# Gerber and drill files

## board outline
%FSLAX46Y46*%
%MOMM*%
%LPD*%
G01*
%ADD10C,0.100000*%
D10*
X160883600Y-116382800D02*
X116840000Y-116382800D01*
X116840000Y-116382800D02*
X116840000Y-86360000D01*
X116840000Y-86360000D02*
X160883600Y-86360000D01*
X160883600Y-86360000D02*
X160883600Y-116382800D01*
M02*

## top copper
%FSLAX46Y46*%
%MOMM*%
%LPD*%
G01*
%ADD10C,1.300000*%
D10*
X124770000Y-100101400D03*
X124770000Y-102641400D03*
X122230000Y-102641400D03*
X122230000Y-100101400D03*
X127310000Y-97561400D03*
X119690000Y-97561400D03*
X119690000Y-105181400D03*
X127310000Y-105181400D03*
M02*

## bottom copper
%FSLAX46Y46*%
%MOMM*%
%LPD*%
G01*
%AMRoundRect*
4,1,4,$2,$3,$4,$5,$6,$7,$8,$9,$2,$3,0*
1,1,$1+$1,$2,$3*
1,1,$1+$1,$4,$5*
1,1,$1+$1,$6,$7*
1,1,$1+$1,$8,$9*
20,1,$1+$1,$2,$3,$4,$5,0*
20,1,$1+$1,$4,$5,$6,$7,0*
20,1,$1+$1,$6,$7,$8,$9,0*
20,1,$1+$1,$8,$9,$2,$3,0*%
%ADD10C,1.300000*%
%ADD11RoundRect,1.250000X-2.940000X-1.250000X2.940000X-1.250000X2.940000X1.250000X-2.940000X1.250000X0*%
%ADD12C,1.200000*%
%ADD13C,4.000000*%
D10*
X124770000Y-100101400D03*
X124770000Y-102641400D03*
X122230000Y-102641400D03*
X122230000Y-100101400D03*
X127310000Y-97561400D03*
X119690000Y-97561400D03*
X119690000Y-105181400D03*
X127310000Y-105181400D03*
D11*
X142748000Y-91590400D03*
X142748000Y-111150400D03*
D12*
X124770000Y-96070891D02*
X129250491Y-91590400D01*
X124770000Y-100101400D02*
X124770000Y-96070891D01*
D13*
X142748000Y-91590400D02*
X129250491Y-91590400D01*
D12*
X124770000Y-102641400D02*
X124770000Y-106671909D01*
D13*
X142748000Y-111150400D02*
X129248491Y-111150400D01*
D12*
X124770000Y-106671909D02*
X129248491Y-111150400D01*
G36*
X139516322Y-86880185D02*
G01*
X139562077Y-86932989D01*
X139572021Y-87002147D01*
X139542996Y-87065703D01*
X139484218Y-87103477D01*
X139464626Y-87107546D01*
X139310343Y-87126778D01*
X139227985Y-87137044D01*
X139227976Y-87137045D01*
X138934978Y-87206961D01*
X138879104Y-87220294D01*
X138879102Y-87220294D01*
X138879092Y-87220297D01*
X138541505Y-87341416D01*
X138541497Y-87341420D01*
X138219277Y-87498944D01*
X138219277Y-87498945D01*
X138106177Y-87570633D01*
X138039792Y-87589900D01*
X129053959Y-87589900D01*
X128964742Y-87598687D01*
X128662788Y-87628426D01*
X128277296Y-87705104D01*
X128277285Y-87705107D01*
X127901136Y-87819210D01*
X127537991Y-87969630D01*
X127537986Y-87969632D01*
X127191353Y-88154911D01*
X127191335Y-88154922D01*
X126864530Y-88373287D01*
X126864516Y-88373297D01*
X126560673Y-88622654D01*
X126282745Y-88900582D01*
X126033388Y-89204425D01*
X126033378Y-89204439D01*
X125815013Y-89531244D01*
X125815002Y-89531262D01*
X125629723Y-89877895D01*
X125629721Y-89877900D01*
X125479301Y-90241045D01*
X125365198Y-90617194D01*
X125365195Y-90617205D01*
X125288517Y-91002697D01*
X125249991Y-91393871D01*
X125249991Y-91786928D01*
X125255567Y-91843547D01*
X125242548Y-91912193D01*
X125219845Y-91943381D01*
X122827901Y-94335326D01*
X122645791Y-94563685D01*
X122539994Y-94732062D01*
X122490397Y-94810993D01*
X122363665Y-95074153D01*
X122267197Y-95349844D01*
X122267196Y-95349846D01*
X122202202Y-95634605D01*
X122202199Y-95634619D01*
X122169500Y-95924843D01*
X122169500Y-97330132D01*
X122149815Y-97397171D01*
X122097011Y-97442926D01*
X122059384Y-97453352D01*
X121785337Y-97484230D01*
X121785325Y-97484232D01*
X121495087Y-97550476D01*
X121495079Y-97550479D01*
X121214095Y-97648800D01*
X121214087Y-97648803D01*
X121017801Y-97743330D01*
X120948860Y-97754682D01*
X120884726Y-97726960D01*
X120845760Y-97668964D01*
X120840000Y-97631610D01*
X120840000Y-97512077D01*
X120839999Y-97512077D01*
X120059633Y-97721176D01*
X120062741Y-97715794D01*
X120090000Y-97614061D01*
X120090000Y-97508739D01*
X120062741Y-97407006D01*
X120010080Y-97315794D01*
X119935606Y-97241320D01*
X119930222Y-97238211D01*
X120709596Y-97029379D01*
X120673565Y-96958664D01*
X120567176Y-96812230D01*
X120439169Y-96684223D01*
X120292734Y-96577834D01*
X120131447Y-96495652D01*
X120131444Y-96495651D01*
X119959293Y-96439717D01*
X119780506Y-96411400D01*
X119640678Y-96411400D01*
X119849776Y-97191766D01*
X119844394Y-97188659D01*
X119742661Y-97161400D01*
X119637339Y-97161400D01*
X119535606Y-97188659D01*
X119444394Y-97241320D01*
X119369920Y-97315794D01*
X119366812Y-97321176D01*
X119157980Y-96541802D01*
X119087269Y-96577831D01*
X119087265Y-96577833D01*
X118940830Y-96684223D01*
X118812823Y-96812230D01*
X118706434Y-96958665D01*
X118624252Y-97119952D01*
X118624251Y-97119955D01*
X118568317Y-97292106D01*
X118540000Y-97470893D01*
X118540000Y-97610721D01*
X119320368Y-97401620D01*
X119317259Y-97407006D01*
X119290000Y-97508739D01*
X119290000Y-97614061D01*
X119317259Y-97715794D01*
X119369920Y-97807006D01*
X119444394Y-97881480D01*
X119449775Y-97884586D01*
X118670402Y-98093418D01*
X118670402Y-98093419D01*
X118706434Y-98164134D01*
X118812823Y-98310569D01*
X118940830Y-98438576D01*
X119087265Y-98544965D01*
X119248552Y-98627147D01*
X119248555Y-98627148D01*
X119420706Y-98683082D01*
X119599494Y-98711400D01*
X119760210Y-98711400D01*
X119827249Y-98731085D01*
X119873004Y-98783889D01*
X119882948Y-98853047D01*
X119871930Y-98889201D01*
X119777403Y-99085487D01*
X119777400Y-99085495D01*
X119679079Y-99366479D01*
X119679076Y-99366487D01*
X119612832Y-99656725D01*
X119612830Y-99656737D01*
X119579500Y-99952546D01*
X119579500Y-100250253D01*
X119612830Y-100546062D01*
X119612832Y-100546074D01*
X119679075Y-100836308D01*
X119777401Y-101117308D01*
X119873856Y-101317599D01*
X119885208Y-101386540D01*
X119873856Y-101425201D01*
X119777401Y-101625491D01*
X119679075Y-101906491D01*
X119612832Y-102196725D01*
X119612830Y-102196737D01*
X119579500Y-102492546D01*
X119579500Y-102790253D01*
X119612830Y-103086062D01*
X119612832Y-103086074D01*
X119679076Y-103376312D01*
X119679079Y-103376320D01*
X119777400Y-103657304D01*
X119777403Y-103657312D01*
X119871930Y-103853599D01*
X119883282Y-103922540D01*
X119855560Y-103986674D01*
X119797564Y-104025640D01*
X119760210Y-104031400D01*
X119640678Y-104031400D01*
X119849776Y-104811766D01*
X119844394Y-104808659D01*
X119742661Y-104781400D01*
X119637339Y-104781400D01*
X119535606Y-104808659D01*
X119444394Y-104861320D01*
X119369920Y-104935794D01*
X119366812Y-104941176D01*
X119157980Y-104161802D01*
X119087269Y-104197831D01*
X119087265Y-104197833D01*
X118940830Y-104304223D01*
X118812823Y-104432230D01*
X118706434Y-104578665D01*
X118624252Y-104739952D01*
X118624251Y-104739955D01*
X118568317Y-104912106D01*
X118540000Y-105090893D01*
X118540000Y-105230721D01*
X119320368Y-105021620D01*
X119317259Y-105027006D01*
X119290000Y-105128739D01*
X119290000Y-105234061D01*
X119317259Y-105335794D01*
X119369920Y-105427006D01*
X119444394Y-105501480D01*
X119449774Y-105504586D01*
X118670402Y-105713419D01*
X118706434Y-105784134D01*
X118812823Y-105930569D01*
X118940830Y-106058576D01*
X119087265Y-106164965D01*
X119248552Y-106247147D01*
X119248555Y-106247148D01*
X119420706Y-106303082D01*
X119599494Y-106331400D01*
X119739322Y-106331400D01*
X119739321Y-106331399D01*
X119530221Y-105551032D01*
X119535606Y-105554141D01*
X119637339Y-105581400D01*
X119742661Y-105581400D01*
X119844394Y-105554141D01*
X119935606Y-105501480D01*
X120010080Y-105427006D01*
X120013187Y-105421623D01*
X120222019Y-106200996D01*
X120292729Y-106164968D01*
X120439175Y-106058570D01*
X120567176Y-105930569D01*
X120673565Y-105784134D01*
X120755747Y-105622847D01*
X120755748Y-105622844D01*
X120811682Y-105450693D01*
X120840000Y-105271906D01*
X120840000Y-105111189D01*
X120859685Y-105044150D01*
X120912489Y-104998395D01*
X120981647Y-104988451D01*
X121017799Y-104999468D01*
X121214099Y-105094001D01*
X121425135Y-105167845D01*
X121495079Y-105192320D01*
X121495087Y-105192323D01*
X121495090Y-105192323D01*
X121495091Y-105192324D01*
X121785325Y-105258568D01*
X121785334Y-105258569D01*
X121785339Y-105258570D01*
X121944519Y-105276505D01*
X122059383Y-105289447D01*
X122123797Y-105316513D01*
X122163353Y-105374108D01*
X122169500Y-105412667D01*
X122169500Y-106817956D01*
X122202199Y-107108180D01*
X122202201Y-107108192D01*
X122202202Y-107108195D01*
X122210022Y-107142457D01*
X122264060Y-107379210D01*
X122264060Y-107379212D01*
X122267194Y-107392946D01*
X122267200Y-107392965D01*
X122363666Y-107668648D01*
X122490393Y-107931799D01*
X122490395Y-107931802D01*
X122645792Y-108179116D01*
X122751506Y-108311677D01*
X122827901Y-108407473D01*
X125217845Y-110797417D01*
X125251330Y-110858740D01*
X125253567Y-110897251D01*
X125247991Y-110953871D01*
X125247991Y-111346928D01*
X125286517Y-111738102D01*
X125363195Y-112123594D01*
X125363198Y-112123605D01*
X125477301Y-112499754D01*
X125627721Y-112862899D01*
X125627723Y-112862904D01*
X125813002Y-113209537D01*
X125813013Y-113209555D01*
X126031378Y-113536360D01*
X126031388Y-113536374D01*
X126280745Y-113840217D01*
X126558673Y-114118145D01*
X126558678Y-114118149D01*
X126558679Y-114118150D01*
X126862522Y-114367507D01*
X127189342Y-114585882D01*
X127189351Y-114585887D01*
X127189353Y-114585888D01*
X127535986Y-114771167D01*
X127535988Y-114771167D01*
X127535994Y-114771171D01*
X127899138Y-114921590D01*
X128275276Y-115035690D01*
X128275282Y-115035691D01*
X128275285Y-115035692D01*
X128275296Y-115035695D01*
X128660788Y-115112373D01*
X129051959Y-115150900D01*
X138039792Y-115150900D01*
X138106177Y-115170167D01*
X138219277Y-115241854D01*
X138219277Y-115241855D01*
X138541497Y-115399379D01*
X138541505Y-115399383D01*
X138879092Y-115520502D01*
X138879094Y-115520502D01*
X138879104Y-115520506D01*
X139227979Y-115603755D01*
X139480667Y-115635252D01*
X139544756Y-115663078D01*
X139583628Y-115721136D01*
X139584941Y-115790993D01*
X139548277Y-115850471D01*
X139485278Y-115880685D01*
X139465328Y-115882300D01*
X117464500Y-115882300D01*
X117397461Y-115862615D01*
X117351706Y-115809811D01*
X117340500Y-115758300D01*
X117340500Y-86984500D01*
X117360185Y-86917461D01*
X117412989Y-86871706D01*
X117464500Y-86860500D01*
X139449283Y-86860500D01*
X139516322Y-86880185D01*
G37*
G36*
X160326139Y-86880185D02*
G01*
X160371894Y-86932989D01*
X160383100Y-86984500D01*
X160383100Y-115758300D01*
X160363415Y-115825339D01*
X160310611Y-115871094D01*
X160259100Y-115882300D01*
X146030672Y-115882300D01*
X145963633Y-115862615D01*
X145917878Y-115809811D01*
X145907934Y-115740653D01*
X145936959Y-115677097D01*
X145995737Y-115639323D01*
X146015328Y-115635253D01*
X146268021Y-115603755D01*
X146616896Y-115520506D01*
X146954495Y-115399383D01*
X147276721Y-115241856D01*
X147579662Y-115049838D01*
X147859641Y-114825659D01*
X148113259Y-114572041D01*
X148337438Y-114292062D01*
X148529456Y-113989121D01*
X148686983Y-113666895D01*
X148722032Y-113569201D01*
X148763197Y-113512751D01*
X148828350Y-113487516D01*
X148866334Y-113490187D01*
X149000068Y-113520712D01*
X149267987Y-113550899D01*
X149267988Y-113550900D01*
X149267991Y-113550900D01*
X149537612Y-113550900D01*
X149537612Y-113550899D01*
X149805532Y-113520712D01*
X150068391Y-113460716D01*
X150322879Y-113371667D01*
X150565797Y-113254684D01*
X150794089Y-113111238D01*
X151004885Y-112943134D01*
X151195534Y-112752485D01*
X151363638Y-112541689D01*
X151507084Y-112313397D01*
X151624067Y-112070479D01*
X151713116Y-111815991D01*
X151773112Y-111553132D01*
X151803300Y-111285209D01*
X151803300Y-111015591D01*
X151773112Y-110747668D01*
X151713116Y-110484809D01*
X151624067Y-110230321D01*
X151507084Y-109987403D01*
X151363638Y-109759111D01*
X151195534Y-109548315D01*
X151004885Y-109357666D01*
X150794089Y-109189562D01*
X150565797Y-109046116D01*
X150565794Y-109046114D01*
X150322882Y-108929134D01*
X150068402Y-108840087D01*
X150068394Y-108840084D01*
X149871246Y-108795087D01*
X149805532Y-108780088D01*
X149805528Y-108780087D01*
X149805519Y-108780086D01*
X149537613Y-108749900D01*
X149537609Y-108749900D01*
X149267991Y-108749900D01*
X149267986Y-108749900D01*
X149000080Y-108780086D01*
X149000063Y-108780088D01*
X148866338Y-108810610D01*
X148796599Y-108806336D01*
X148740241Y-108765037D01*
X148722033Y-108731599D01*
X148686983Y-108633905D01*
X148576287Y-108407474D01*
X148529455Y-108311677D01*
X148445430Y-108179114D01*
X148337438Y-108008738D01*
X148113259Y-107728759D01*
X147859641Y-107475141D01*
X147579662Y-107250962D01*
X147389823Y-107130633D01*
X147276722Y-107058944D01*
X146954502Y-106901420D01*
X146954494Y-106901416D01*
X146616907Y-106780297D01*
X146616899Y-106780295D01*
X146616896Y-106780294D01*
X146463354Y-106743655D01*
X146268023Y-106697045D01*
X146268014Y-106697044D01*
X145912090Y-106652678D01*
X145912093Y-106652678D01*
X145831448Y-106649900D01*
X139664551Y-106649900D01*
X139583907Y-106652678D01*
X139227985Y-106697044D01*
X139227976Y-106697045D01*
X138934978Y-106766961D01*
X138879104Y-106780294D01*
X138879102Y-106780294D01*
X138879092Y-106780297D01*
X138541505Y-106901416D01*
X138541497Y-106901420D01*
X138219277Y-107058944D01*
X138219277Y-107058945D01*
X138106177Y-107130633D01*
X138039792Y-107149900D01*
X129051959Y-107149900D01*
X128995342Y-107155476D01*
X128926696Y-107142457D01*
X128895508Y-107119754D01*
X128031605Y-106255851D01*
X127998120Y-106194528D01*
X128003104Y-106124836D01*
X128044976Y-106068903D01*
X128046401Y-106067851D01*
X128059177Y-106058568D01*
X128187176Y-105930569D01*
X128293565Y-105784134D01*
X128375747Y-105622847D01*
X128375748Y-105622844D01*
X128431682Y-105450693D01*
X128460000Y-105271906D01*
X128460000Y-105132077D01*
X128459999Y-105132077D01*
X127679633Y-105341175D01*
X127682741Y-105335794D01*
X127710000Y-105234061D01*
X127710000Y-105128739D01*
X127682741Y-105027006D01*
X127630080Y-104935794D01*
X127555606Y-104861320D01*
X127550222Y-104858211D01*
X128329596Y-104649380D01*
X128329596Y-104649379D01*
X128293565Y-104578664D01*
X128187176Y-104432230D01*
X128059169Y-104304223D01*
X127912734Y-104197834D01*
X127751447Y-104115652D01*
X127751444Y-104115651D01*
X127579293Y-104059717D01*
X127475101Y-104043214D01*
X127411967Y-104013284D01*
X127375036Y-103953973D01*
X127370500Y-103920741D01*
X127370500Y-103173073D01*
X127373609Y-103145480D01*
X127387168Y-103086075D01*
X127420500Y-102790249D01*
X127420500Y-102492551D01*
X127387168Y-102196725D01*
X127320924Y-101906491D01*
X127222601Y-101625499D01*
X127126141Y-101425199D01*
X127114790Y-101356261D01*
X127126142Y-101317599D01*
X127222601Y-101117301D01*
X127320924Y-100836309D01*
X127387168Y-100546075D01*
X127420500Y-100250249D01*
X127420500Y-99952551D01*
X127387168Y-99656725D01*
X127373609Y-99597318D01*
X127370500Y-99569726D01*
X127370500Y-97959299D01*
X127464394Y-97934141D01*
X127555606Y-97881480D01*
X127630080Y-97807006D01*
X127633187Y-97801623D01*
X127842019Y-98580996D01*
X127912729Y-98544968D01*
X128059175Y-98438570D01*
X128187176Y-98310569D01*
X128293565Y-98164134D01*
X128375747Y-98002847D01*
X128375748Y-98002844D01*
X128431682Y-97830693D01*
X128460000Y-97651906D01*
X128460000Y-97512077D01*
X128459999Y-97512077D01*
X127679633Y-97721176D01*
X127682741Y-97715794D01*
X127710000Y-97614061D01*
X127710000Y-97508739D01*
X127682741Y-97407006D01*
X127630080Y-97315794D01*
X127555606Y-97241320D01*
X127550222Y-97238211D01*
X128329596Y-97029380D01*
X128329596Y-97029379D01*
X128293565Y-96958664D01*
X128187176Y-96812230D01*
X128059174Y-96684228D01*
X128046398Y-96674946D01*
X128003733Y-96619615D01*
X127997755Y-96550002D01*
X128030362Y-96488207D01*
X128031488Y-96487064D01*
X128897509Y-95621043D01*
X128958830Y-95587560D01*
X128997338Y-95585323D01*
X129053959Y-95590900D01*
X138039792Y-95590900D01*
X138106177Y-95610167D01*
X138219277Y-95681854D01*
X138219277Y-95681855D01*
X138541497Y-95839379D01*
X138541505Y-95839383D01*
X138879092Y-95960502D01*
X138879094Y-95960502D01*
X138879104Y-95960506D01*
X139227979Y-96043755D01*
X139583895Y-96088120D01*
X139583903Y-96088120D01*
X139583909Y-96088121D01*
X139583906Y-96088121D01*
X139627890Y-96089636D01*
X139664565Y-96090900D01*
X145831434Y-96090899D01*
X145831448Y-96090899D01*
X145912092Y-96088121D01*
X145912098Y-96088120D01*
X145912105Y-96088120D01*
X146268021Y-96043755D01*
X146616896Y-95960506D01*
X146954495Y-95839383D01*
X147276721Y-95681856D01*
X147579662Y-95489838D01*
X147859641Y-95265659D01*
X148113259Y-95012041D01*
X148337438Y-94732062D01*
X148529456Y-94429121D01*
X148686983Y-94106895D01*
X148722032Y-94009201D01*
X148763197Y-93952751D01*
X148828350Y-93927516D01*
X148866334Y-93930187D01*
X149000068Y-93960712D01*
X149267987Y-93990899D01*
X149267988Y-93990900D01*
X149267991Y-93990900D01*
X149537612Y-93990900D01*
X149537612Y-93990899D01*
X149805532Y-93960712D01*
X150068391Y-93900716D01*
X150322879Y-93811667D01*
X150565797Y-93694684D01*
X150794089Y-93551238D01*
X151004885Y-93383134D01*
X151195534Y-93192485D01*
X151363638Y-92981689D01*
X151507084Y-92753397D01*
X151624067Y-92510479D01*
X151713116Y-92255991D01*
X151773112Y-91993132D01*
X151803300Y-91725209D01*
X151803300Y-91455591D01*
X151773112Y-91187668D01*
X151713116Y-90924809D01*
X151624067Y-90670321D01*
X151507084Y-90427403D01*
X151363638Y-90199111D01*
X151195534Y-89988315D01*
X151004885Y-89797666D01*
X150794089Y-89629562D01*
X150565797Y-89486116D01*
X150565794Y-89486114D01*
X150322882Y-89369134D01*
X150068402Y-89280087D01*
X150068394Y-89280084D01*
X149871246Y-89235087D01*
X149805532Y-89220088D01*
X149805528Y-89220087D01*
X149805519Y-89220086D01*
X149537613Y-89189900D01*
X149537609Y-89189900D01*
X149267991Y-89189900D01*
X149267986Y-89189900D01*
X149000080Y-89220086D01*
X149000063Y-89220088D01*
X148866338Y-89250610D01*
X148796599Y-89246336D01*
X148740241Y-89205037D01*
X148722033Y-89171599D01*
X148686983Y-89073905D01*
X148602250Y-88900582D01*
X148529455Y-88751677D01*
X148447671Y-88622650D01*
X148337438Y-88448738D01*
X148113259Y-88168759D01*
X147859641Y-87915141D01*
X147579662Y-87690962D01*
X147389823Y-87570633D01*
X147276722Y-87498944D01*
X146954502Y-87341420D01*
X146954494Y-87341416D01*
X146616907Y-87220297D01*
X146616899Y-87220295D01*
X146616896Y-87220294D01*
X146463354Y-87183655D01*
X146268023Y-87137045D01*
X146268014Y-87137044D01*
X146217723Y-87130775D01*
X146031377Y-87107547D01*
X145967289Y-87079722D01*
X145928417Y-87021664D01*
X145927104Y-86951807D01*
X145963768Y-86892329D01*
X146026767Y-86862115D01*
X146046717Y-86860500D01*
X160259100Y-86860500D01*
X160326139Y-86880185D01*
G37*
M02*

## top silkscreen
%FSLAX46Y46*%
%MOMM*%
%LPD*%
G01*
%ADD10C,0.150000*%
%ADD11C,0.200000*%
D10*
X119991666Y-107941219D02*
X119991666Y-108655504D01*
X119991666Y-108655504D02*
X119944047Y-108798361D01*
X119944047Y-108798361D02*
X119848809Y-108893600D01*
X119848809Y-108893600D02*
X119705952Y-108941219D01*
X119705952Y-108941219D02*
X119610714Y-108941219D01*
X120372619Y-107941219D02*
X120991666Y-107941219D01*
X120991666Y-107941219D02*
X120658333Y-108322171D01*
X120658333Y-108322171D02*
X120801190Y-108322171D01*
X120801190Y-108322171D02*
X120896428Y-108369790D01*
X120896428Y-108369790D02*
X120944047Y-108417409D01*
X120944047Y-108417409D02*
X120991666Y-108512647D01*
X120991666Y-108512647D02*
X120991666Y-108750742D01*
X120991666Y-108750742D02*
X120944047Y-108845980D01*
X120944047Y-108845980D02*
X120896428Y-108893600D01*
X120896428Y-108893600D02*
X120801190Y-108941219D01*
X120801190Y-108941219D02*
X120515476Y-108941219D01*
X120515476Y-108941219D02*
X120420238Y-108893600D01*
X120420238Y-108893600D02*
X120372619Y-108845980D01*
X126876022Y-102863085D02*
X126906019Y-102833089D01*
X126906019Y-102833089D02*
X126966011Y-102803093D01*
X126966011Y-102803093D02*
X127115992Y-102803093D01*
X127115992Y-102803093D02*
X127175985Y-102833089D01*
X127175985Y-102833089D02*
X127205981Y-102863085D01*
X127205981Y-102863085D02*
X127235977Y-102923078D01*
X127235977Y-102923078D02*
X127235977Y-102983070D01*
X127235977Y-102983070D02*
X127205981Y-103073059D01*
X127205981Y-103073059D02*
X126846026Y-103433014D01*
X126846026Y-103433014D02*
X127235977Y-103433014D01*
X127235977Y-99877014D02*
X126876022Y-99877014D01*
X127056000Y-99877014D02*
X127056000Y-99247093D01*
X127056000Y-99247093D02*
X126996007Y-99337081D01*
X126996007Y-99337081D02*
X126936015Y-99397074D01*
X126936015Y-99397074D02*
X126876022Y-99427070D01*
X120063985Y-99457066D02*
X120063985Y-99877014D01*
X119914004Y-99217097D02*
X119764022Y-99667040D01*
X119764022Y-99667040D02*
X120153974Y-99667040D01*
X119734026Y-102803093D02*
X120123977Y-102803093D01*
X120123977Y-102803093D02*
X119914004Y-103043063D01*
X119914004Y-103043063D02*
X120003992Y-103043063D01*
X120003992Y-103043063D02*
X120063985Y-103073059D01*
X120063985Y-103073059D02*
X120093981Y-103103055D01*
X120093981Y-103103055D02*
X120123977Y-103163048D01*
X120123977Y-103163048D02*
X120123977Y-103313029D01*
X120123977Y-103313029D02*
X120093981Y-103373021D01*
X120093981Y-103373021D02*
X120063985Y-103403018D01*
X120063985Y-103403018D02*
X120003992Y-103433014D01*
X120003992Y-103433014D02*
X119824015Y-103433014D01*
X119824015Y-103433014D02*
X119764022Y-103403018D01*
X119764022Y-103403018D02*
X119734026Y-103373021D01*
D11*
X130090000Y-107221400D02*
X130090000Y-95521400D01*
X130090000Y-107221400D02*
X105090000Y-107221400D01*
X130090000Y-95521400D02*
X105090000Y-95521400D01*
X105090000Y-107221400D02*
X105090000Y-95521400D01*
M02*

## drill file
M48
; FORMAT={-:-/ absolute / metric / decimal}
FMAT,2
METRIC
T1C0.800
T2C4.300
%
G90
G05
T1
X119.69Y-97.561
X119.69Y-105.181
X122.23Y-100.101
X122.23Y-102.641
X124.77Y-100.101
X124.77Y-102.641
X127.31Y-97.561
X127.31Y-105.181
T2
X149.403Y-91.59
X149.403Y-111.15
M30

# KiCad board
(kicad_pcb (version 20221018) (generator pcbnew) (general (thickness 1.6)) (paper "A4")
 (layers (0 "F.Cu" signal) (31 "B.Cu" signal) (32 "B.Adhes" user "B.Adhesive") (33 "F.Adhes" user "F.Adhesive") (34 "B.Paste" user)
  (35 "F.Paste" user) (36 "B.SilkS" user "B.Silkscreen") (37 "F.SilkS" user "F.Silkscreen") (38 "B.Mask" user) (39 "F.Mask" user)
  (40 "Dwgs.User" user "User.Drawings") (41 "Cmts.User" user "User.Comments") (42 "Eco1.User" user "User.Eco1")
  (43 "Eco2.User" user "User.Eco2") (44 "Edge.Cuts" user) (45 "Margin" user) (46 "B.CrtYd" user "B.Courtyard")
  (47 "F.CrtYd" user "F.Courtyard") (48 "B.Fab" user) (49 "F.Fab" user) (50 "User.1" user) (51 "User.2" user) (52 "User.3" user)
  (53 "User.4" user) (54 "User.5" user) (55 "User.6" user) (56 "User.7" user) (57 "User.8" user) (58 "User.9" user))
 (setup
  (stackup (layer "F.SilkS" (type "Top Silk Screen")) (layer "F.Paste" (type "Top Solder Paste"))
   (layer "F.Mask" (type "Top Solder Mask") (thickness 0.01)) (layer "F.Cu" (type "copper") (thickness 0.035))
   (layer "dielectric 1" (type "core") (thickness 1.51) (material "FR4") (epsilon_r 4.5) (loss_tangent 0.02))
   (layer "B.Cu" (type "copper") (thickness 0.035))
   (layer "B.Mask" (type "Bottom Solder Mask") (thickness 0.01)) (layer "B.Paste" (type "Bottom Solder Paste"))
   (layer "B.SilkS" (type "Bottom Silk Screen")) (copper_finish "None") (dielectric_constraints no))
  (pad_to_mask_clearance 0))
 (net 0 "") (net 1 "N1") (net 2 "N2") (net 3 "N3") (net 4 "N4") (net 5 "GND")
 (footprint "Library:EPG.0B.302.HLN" (layer "F.Cu") (at 123.5 101.3714 180)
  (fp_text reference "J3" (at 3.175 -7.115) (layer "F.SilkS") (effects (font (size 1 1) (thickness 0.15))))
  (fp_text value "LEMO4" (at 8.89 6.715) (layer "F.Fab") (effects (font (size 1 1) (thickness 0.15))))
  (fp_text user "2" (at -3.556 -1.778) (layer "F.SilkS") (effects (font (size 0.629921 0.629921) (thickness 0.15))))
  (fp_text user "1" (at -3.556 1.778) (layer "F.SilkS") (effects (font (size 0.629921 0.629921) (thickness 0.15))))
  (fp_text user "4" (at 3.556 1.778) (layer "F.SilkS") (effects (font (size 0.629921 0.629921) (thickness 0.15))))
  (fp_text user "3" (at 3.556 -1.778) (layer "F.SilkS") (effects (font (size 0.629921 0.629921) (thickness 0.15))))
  (fp_line (start -6.59 -5.85) (end -6.59 5.85) (stroke (width 0.2) (type solid)) (layer "F.SilkS"))
  (fp_line (start -6.59 -5.85) (end 18.41 -5.85) (stroke (width 0.2) (type solid)) (layer "F.SilkS"))
  (fp_line (start -6.59 5.85) (end 18.41 5.85) (stroke (width 0.2) (type solid)) (layer "F.SilkS"))
  (fp_line (start 18.41 -5.85) (end 18.41 5.85) (stroke (width 0.2) (type solid)) (layer "F.SilkS"))
  (pad "1" thru_hole circle (at -1.27 1.27 60) (size 1.3 1.3) (drill 0.8) (layers "*.Cu" "*.Mask") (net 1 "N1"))
  (pad "2" thru_hole circle (at -1.27 -1.27 60) (size 1.3 1.3) (drill 0.8) (layers "*.Cu" "*.Mask") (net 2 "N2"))
  (pad "3" thru_hole circle (at 1.27 -1.27 60) (size 1.3 1.3) (drill 0.8) (layers "*.Cu" "*.Mask") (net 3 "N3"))
  (pad "4" thru_hole circle (at 1.27 1.27 60) (size 1.3 1.3) (drill 0.8) (layers "*.Cu" "*.Mask") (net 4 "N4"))
  (pad "5" thru_hole circle (at -3.81 3.81 60) (size 1.3 1.3) (drill 0.8) (layers "*.Cu" "*.Mask") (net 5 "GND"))
  (pad "6" thru_hole circle (at 3.81 3.81 60) (size 1.3 1.3) (drill 0.8) (layers "*.Cu" "*.Mask") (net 5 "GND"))
  (pad "7" thru_hole circle (at 3.81 -3.81 60) (size 1.3 1.3) (drill 0.8) (layers "*.Cu" "*.Mask") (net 5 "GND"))
  (pad "8" thru_hole circle (at -3.81 -3.81 60) (size 1.3 1.3) (drill 0.8) (layers "*.Cu" "*.Mask") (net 5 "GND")))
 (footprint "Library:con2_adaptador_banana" (layer "B.Cu") (at 146.9644 91.5904)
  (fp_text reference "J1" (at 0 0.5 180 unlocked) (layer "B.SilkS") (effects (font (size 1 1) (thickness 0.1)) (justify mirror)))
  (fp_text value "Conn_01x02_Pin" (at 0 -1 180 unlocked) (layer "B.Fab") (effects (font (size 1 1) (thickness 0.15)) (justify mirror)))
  (pad "" np_thru_hole circle (at 2.4384 0) (size 4.1 4.1) (drill 4.3) (layers "F&B.Cu" "*.Mask"))
  (pad "" np_thru_hole circle (at 2.4384 19.56) (size 4.1 4.1) (drill 4.3) (layers "F&B.Cu" "*.Mask"))
  (pad "1" smd roundrect (at -4.2164 0) (size 8.38 5) (layers "B.Cu" "B.Paste" "B.Mask") (roundrect_rratio 0.25) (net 1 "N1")
   (thermal_bridge_angle 45))
  (pad "2" smd roundrect (at -4.2164 19.56) (size 8.38 5) (layers "B.Cu" "B.Paste" "B.Mask") (roundrect_rratio 0.25) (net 2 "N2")
   (thermal_bridge_angle 45)))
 (gr_line (start 160.8836 116.3828) (end 116.84 116.3828) (stroke (width 0.1) (type default)) (layer "Edge.Cuts"))
 (gr_line (start 116.84 116.3828) (end 116.84 86.36) (stroke (width 0.1) (type default)) (layer "Edge.Cuts"))
 (gr_line (start 116.84 86.36) (end 160.8836 86.36) (stroke (width 0.1) (type default)) (layer "Edge.Cuts"))
 (gr_line (start 160.8836 86.36) (end 160.8836 116.3828) (stroke (width 0.1) (type default)) (layer "Edge.Cuts"))
 (segment (start 124.77 96.070891) (end 129.250491 91.5904) (width 1.2) (layer "B.Cu") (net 1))
 (segment (start 124.77 100.1014) (end 124.77 96.070891) (width 1.2) (layer "B.Cu") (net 1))
 (segment (start 142.748 91.5904) (end 129.250491 91.5904) (width 4) (layer "B.Cu") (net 1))
 (segment (start 124.77 102.6414) (end 124.77 106.671909) (width 1.2) (layer "B.Cu") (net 2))
 (segment (start 142.748 111.1504) (end 129.248491 111.1504) (width 4) (layer "B.Cu") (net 2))
 (segment (start 124.77 106.671909) (end 129.248491 111.1504) (width 1.2) (layer "B.Cu") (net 2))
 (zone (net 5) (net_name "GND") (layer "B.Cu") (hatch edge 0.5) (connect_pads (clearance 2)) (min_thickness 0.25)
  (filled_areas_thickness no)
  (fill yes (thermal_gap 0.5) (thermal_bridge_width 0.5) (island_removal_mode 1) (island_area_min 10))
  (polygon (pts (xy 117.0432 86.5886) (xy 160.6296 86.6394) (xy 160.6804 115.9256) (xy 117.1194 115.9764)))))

